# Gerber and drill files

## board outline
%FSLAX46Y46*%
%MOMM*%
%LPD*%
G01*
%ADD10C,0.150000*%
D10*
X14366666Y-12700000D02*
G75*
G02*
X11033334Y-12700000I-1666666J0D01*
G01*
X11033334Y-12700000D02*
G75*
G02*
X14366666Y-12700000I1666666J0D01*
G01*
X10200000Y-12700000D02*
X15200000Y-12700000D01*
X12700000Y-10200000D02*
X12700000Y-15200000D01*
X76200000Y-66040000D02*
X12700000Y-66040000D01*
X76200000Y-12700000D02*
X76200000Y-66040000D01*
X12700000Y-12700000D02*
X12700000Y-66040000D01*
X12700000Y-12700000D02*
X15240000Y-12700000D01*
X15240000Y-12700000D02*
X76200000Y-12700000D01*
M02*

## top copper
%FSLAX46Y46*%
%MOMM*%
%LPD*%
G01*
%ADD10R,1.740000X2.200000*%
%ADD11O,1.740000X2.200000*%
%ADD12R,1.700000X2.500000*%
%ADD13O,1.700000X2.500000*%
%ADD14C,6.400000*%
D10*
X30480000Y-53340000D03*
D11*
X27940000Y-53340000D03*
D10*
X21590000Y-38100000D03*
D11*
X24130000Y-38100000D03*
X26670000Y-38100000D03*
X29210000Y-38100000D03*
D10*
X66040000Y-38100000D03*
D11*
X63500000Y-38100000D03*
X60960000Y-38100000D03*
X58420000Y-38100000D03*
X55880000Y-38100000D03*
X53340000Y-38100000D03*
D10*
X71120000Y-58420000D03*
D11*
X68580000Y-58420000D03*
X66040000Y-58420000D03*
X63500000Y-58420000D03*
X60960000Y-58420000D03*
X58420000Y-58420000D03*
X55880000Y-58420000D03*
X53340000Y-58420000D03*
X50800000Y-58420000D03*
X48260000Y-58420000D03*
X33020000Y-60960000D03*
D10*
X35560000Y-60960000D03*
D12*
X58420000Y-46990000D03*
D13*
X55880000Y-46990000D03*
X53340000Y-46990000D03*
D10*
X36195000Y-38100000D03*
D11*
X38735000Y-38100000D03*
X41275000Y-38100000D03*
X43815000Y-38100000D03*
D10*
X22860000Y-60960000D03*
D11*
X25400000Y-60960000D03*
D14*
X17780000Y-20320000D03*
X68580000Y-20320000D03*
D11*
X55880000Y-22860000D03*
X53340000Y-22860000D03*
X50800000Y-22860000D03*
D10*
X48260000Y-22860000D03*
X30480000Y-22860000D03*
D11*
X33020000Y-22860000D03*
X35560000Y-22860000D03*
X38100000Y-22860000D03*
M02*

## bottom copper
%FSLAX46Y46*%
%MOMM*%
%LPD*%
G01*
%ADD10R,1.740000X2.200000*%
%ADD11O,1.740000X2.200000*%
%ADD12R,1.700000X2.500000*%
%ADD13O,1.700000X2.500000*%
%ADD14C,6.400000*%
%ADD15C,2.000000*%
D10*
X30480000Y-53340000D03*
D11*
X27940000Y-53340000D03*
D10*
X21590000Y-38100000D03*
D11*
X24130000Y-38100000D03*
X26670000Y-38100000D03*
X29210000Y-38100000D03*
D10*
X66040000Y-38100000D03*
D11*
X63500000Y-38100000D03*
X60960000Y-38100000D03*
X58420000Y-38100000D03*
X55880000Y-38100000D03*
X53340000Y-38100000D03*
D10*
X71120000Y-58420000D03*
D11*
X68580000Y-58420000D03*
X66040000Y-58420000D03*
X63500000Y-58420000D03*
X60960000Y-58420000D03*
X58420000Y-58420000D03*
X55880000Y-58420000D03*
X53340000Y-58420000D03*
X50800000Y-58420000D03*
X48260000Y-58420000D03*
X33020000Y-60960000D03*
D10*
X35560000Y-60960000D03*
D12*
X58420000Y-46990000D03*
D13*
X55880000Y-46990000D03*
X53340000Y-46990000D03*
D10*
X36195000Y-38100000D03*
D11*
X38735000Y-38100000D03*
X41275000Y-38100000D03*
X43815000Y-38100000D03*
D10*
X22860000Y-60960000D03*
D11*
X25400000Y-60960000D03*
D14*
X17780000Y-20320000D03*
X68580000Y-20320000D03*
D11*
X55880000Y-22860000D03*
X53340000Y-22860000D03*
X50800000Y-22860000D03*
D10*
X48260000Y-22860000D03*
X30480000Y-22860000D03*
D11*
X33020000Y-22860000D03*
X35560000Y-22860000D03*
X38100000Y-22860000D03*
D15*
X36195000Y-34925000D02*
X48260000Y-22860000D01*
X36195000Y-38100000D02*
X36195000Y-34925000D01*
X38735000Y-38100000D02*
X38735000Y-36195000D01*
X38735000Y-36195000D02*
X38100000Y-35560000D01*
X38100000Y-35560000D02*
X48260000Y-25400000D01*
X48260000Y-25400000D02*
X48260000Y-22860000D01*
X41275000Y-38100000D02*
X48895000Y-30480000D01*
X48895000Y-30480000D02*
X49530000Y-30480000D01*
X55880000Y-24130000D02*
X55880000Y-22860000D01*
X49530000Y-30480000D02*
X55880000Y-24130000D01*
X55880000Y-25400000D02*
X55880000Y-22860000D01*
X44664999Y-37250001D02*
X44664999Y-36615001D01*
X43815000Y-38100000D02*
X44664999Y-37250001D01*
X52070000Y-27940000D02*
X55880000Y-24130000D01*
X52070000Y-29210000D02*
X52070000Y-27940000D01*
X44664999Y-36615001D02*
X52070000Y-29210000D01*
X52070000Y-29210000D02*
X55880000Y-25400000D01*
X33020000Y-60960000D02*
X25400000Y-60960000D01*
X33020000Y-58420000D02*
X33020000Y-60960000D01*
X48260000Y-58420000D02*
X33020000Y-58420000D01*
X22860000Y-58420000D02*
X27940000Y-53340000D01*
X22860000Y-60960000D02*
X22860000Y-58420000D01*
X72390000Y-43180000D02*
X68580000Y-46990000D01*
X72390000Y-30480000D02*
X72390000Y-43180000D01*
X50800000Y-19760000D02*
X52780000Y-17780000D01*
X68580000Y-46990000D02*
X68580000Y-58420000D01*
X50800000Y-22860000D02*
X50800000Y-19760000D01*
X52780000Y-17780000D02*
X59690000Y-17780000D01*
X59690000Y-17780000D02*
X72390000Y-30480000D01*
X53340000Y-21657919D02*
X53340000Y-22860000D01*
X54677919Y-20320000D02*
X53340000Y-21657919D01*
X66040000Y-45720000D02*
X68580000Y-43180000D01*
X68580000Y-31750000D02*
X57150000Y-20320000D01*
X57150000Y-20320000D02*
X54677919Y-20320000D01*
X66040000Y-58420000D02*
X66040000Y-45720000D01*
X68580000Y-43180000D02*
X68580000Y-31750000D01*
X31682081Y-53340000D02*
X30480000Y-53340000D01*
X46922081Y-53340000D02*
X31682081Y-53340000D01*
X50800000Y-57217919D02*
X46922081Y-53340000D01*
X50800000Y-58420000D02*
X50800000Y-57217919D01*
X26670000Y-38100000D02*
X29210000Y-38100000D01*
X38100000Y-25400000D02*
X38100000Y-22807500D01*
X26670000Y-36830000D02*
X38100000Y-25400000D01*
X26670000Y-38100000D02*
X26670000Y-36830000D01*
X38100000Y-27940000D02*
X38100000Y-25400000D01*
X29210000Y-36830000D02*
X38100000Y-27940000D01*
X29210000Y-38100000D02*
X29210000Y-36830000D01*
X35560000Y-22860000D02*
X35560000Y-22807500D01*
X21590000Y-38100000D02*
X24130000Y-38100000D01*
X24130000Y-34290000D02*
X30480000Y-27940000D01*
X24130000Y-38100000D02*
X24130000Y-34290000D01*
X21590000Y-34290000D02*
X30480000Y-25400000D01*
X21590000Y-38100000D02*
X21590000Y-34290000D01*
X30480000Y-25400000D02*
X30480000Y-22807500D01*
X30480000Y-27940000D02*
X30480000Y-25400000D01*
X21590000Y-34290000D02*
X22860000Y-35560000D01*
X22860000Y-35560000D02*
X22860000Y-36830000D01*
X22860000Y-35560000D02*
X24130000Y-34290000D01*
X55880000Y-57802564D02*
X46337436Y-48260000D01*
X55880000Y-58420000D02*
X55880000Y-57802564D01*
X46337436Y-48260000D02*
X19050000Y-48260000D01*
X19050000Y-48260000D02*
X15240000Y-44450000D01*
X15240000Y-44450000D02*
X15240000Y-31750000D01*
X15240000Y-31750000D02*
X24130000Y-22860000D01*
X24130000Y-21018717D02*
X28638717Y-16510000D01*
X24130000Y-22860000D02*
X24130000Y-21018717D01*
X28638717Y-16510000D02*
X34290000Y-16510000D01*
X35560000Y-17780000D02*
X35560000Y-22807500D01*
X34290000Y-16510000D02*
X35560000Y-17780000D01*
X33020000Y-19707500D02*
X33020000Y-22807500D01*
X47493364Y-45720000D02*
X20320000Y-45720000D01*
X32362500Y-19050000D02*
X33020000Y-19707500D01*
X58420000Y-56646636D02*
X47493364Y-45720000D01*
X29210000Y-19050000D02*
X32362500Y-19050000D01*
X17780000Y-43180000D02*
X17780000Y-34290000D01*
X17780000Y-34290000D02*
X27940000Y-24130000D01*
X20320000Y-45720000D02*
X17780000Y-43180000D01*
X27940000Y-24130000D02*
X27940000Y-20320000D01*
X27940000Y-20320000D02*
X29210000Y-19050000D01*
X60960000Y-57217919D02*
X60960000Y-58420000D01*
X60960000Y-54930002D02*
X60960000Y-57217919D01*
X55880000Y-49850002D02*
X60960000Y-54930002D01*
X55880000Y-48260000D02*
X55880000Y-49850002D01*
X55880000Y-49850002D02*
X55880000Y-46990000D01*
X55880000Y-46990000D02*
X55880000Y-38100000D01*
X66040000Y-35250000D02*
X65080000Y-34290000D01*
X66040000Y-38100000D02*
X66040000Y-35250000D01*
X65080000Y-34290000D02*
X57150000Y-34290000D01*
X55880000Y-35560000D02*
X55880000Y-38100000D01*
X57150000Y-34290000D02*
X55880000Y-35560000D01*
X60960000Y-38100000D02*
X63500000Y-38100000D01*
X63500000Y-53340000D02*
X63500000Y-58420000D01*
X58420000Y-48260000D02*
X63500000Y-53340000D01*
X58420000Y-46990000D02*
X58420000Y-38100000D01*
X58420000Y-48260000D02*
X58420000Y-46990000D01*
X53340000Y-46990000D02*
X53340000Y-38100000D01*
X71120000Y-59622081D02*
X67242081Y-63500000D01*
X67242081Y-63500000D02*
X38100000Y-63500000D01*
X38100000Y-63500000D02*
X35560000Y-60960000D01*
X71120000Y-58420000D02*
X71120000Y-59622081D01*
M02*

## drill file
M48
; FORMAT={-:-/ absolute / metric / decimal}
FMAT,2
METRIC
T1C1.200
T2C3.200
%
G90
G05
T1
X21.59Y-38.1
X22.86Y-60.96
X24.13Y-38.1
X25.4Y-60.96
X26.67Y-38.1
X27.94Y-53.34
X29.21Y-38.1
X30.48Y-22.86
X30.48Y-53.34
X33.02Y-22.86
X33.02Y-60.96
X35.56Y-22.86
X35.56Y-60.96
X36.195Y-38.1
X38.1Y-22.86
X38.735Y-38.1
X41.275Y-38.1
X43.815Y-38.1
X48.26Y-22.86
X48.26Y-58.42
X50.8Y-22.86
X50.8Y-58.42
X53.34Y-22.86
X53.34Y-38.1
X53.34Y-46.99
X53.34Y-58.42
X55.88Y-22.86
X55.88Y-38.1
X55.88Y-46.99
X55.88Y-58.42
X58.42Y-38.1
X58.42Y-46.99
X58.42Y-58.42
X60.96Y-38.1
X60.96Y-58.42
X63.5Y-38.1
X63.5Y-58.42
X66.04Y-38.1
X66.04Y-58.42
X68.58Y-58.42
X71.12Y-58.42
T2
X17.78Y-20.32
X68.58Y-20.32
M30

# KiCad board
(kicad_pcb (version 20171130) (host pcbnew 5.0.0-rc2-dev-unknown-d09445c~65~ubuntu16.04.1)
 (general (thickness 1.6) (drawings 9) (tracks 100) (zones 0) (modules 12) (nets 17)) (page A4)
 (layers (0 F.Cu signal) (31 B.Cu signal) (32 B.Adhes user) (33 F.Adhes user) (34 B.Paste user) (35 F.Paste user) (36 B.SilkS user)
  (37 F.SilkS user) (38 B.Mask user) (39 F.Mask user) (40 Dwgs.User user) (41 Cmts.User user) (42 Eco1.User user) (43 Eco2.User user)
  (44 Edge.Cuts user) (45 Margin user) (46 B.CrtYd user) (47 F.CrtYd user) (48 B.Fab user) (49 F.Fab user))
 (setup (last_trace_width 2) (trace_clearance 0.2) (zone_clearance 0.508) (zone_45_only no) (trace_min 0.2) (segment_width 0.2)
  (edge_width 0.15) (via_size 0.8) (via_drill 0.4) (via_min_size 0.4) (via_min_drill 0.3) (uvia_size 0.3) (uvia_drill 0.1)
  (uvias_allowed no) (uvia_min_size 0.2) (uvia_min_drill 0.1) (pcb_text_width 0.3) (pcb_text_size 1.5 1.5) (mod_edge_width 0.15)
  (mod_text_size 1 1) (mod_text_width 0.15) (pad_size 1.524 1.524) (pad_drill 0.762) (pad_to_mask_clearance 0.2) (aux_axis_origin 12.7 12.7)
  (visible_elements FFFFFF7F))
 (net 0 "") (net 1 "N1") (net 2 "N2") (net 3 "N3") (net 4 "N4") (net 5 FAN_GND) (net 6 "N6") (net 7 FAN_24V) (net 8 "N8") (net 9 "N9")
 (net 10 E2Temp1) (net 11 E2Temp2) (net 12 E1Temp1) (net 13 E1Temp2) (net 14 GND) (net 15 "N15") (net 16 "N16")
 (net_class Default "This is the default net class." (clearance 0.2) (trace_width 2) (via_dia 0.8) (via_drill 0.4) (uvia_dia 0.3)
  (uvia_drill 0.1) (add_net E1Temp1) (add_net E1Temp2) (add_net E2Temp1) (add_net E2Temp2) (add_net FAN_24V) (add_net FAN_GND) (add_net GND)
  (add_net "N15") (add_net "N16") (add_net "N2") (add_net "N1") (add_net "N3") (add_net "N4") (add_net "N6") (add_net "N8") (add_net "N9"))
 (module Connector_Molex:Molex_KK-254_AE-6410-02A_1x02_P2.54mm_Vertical (layer F.Cu) (at 30.48 53.34 180)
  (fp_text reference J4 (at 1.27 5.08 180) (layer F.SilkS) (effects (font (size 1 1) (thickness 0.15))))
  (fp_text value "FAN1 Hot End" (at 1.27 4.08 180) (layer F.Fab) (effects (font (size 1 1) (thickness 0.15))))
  (pad 1 thru_hole rect (at 0 0 180) (size 1.74 2.2) (drill 1.2) (layers *.Cu *.Mask) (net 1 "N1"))
  (pad 2 thru_hole oval (at 2.54 0 180) (size 1.74 2.2) (drill 1.2) (layers *.Cu *.Mask) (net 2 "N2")))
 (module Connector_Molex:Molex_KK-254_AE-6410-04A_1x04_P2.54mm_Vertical (layer F.Cu) (at 21.59 38.1)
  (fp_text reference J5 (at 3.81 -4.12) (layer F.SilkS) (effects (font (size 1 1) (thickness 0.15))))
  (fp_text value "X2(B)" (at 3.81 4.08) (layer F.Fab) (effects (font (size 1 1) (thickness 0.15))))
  (pad 1 thru_hole rect (at 0 0) (size 1.74 2.2) (drill 1.2) (layers *.Cu *.Mask) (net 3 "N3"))
  (pad 2 thru_hole oval (at 2.54 0) (size 1.74 2.2) (drill 1.2) (layers *.Cu *.Mask) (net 3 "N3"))
  (pad 3 thru_hole oval (at 5.08 0) (size 1.74 2.2) (drill 1.2) (layers *.Cu *.Mask) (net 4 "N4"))
  (pad 4 thru_hole oval (at 7.62 0) (size 1.74 2.2) (drill 1.2) (layers *.Cu *.Mask) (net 4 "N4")))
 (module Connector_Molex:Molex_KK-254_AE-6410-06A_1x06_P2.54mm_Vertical (layer F.Cu) (at 66.04 38.1 180)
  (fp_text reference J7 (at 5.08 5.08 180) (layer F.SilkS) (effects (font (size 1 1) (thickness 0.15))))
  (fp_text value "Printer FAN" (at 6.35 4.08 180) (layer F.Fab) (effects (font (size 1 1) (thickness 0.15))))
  (pad 1 thru_hole rect (at 0 0 180) (size 1.74 2.2) (drill 1.2) (layers *.Cu *.Mask) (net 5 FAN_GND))
  (pad 2 thru_hole oval (at 2.54 0 180) (size 1.74 2.2) (drill 1.2) (layers *.Cu *.Mask) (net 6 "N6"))
  (pad 3 thru_hole oval (at 5.08 0 180) (size 1.74 2.2) (drill 1.2) (layers *.Cu *.Mask) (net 6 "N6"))
  (pad 4 thru_hole oval (at 7.62 0 180) (size 1.74 2.2) (drill 1.2) (layers *.Cu *.Mask) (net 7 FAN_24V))
  (pad 5 thru_hole oval (at 10.16 0 180) (size 1.74 2.2) (drill 1.2) (layers *.Cu *.Mask) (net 5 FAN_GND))
  (pad 6 thru_hole oval (at 12.7 0 180) (size 1.74 2.2) (drill 1.2) (layers *.Cu *.Mask) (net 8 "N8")))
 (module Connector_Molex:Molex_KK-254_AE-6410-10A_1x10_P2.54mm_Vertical (layer F.Cu) (at 71.12 58.42 180)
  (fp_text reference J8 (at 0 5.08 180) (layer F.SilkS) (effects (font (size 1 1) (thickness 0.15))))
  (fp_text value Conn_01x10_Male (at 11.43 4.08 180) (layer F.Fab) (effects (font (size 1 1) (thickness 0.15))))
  (pad 1 thru_hole rect (at 0 0 180) (size 1.74 2.2) (drill 1.2) (layers *.Cu *.Mask) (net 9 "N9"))
  (pad 2 thru_hole oval (at 2.54 0 180) (size 1.74 2.2) (drill 1.2) (layers *.Cu *.Mask) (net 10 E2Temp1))
  (pad 3 thru_hole oval (at 5.08 0 180) (size 1.74 2.2) (drill 1.2) (layers *.Cu *.Mask) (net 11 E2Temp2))
  (pad 4 thru_hole oval (at 7.62 0 180) (size 1.74 2.2) (drill 1.2) (layers *.Cu *.Mask) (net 7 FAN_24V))
  (pad 5 thru_hole oval (at 10.16 0 180) (size 1.74 2.2) (drill 1.2) (layers *.Cu *.Mask) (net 5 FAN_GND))
  (pad 6 thru_hole oval (at 12.7 0 180) (size 1.74 2.2) (drill 1.2) (layers *.Cu *.Mask) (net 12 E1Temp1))
  (pad 7 thru_hole oval (at 15.24 0 180) (size 1.74 2.2) (drill 1.2) (layers *.Cu *.Mask) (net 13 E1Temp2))
  (pad 8 thru_hole oval (at 17.78 0 180) (size 1.74 2.2) (drill 1.2) (layers *.Cu *.Mask))
  (pad 9 thru_hole oval (at 20.32 0 180) (size 1.74 2.2) (drill 1.2) (layers *.Cu *.Mask) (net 1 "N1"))
  (pad 10 thru_hole oval (at 22.86 0 180) (size 1.74 2.2) (drill 1.2) (layers *.Cu *.Mask) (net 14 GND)))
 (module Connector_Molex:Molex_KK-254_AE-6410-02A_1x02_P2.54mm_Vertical (layer F.Cu) (at 35.56 60.96 180)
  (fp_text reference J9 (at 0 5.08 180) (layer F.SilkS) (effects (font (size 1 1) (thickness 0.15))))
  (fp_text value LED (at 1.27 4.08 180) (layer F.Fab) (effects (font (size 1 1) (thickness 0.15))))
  (pad 2 thru_hole oval (at 2.54 0 180) (size 1.74 2.2) (drill 1.2) (layers *.Cu *.Mask) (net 14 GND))
  (pad 1 thru_hole rect (at 0 0 180) (size 1.74 2.2) (drill 1.2) (layers *.Cu *.Mask) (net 9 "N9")))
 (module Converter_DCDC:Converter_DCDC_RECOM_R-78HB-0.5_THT (layer F.Cu) (at 58.42 46.99 180)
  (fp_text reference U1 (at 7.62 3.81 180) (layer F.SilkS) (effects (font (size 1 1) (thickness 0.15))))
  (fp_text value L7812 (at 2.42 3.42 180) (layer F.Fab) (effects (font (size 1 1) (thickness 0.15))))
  (pad 1 thru_hole rect (at 0 0 180) (size 1.7 2.5) (drill 1.2) (layers *.Cu *.Mask) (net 7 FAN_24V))
  (pad 2 thru_hole oval (at 2.54 0 180) (size 1.7 2.5) (drill 1.2) (layers *.Cu *.Mask) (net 5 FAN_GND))
  (pad 3 thru_hole oval (at 5.08 0 180) (size 1.7 2.5) (drill 1.2) (layers *.Cu *.Mask) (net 8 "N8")))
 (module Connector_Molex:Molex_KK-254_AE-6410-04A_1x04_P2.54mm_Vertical (layer F.Cu) (at 36.195 38.1)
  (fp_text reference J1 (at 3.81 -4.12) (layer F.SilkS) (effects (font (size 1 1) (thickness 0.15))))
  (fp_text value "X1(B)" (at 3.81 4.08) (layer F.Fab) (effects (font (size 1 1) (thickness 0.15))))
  (pad 1 thru_hole rect (at 0 0) (size 1.74 2.2) (drill 1.2) (layers *.Cu *.Mask) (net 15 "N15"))
  (pad 2 thru_hole oval (at 2.54 0) (size 1.74 2.2) (drill 1.2) (layers *.Cu *.Mask) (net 15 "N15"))
  (pad 3 thru_hole oval (at 5.08 0) (size 1.74 2.2) (drill 1.2) (layers *.Cu *.Mask) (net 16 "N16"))
  (pad 4 thru_hole oval (at 7.62 0) (size 1.74 2.2) (drill 1.2) (layers *.Cu *.Mask) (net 16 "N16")))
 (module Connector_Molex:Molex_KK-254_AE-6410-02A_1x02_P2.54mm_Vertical (layer F.Cu) (at 22.86 60.96)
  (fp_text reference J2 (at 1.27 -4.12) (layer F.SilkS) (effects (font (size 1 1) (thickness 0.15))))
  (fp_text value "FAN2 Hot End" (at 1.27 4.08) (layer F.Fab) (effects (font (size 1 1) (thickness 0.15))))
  (pad 1 thru_hole rect (at 0 0) (size 1.74 2.2) (drill 1.2) (layers *.Cu *.Mask) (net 2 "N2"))
  (pad 2 thru_hole oval (at 2.54 0) (size 1.74 2.2) (drill 1.2) (layers *.Cu *.Mask) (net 14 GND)))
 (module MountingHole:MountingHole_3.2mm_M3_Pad (layer F.Cu) (at 17.78 20.32)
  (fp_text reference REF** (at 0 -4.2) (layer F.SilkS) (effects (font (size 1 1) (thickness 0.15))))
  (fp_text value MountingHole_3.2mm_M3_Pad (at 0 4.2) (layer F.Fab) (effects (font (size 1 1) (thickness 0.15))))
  (pad 1 thru_hole circle (at 0 0) (size 6.4 6.4) (drill 3.2) (layers *.Cu *.Mask)))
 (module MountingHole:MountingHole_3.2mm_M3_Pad (layer F.Cu) (at 68.58 20.32)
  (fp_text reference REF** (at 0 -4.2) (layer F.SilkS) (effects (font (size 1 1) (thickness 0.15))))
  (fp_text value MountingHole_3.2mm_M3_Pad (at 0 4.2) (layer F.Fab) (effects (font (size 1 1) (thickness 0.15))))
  (pad 1 thru_hole circle (at 0 0) (size 6.4 6.4) (drill 3.2) (layers *.Cu *.Mask)))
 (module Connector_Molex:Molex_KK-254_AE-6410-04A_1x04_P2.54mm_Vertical (layer F.Cu) (at 48.26 22.86)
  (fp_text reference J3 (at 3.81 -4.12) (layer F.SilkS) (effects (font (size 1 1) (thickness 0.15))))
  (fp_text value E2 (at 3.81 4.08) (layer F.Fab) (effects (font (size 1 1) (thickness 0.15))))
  (pad 4 thru_hole oval (at 7.62 0) (size 1.74 2.2) (drill 1.2) (layers *.Cu *.Mask) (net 16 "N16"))
  (pad 3 thru_hole oval (at 5.08 0) (size 1.74 2.2) (drill 1.2) (layers *.Cu *.Mask) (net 11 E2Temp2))
  (pad 2 thru_hole oval (at 2.54 0) (size 1.74 2.2) (drill 1.2) (layers *.Cu *.Mask) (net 10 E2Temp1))
  (pad 1 thru_hole rect (at 0 0) (size 1.74 2.2) (drill 1.2) (layers *.Cu *.Mask) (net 15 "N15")))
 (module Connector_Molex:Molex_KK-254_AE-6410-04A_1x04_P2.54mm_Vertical (layer F.Cu) (at 30.48 22.86)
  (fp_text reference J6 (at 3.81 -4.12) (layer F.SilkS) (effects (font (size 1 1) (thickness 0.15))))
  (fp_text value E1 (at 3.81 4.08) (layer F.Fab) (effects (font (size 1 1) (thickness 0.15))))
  (pad 1 thru_hole rect (at 0 0) (size 1.74 2.2) (drill 1.2) (layers *.Cu *.Mask) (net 3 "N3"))
  (pad 2 thru_hole oval (at 2.54 0) (size 1.74 2.2) (drill 1.2) (layers *.Cu *.Mask) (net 12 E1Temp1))
  (pad 3 thru_hole oval (at 5.08 0) (size 1.74 2.2) (drill 1.2) (layers *.Cu *.Mask) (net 13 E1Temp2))
  (pad 4 thru_hole oval (at 7.62 0) (size 1.74 2.2) (drill 1.2) (layers *.Cu *.Mask) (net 4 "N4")))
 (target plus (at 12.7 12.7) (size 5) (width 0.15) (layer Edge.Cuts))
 (gr_line (start 76.2 66.04) (end 12.7 66.04) (layer Edge.Cuts) (width 0.15))
 (gr_line (start 76.2 12.7) (end 76.2 66.04) (layer Edge.Cuts) (width 0.15))
 (gr_line (start 12.7 12.7) (end 12.7 66.04) (layer Edge.Cuts) (width 0.15))
 (gr_line (start 12.7 12.7) (end 15.24 12.7) (layer Edge.Cuts) (width 0.15))
 (gr_line (start 15.24 12.7) (end 76.2 12.7) (layer Edge.Cuts) (width 0.15))
 (segment (start 36.195 34.925) (end 48.26 22.86) (width 2) (layer B.Cu) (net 15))
 (segment (start 36.195 38.1) (end 36.195 34.925) (width 2) (layer B.Cu) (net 15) (status 10))
 (segment (start 38.735 38.1) (end 38.735 36.195) (width 2) (layer B.Cu) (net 15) (status 10))
 (segment (start 38.735 36.195) (end 38.1 35.56) (width 2) (layer B.Cu) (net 15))
 (segment (start 38.1 35.56) (end 48.26 25.4) (width 2) (layer B.Cu) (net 15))
 (segment (start 48.26 25.4) (end 48.26 22.86) (width 2) (layer B.Cu) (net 15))
 (segment (start 41.275 38.1) (end 48.895 30.48) (width 2) (layer B.Cu) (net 16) (status 10))
 (segment (start 48.895 30.48) (end 49.53 30.48) (width 2) (layer B.Cu) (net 16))
 (segment (start 55.88 24.13) (end 55.88 22.86) (width 2) (layer B.Cu) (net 16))
 (segment (start 49.53 30.48) (end 55.88 24.13) (width 2) (layer B.Cu) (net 16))
 (segment (start 55.88 25.4) (end 55.88 22.86) (width 2) (layer B.Cu) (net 16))
 (segment (start 44.664999 37.250001) (end 44.664999 36.615001) (width 2) (layer B.Cu) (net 16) (status 10))
 (segment (start 43.815 38.1) (end 44.664999 37.250001) (width 2) (layer B.Cu) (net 16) (status 30))
 (segment (start 52.07 27.94) (end 55.88 24.13) (width 2) (layer B.Cu) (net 16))
 (segment (start 52.07 29.21) (end 52.07 27.94) (width 2) (layer B.Cu) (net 16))
 (segment (start 44.664999 36.615001) (end 52.07 29.21) (width 2) (layer B.Cu) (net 16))
 (segment (start 52.07 29.21) (end 55.88 25.4) (width 2) (layer B.Cu) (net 16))
 (segment (start 33.02 60.96) (end 25.4 60.96) (width 2) (layer B.Cu) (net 14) (status 30))
 (segment (start 33.02 58.42) (end 33.02 60.96) (width 2) (layer B.Cu) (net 14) (status 20))
 (segment (start 48.26 58.42) (end 33.02 58.42) (width 2) (layer B.Cu) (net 14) (status 10))
 (segment (start 22.86 58.42) (end 27.94 53.34) (width 2) (layer B.Cu) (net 2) (status 20))
 (segment (start 22.86 60.96) (end 22.86 58.42) (width 2) (layer B.Cu) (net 2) (status 10))
 (segment (start 72.39 43.18) (end 68.58 46.99) (width 2) (layer B.Cu) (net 10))
 (segment (start 72.39 30.48) (end 72.39 43.18) (width 2) (layer B.Cu) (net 10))
 (segment (start 50.8 19.76) (end 52.78 17.78) (width 2) (layer B.Cu) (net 10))
 (segment (start 68.58 46.99) (end 68.58 58.42) (width 2) (layer B.Cu) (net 10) (status 20))
 (segment (start 50.8 22.86) (end 50.8 19.76) (width 2) (layer B.Cu) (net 10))
 (segment (start 52.78 17.78) (end 59.69 17.78) (width 2) (layer B.Cu) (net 10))
 (segment (start 59.69 17.78) (end 72.39 30.48) (width 2) (layer B.Cu) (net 10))
 (segment (start 53.34 21.657919) (end 53.34 22.86) (width 2) (layer B.Cu) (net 11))
 (segment (start 54.677919 20.32) (end 53.34 21.657919) (width 2) (layer B.Cu) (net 11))
 (segment (start 66.04 45.72) (end 68.58 43.18) (width 2) (layer B.Cu) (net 11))
 (segment (start 68.58 31.75) (end 57.15 20.32) (width 2) (layer B.Cu) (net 11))
 (segment (start 57.15 20.32) (end 54.677919 20.32) (width 2) (layer B.Cu) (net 11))
 (segment (start 66.04 58.42) (end 66.04 45.72) (width 2) (layer B.Cu) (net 11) (status 10))
 (segment (start 68.58 43.18) (end 68.58 31.75) (width 2) (layer B.Cu) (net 11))
 (segment (start 31.682081 53.34) (end 30.48 53.34) (width 2) (layer B.Cu) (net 1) (status 20))
 (segment (start 46.922081 53.34) (end 31.682081 53.34) (width 2) (layer B.Cu) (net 1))
 (segment (start 50.8 57.217919) (end 46.922081 53.34) (width 2) (layer B.Cu) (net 1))
 (segment (start 50.8 58.42) (end 50.8 57.217919) (width 2) (layer B.Cu) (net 1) (status 10))
 (segment (start 26.67 38.1) (end 29.21 38.1) (width 2) (layer B.Cu) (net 4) (status 30))
 (segment (start 38.1 25.4) (end 38.1 22.8075) (width 2) (layer B.Cu) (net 4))
 (segment (start 26.67 36.83) (end 38.1 25.4) (width 2) (layer B.Cu) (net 4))
 (segment (start 26.67 38.1) (end 26.67 36.83) (width 2) (layer B.Cu) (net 4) (status 10))
 (segment (start 38.1 27.94) (end 38.1 25.4) (width 2) (layer B.Cu) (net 4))
 (segment (start 29.21 36.83) (end 38.1 27.94) (width 2) (layer B.Cu) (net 4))
 (segment (start 29.21 38.1) (end 29.21 36.83) (width 2) (layer B.Cu) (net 4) (status 10))
 (segment (start 35.56 22.86) (end 35.56 22.8075) (width 2) (layer B.Cu) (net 13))
 (segment (start 21.59 38.1) (end 24.13 38.1) (width 2) (layer B.Cu) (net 3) (status 30))
 (segment (start 24.13 34.29) (end 30.48 27.94) (width 2) (layer B.Cu) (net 3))
 (segment (start 24.13 38.1) (end 24.13 34.29) (width 2) (layer B.Cu) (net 3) (status 10))
 (segment (start 21.59 34.29) (end 30.48 25.4) (width 2) (layer B.Cu) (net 3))
 (segment (start 21.59 38.1) (end 21.59 34.29) (width 2) (layer B.Cu) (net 3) (status 10))
 (segment (start 30.48 25.4) (end 30.48 22.8075) (width 2) (layer B.Cu) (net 3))
 (segment (start 30.48 27.94) (end 30.48 25.4) (width 2) (layer B.Cu) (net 3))
 (segment (start 21.59 34.29) (end 22.86 35.56) (width 2) (layer B.Cu) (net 3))
 (segment (start 22.86 35.56) (end 22.86 36.83) (width 2) (layer B.Cu) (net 3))
 (segment (start 22.86 35.56) (end 24.13 34.29) (width 2) (layer B.Cu) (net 3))
 (segment (start 55.88 57.802564) (end 46.337436 48.26) (width 2) (layer B.Cu) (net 13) (status 10))
 (segment (start 55.88 58.42) (end 55.88 57.802564) (width 2) (layer B.Cu) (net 13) (status 30))
 (segment (start 46.337436 48.26) (end 19.05 48.26) (width 2) (layer B.Cu) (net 13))
 (segment (start 19.05 48.26) (end 15.24 44.45) (width 2) (layer B.Cu) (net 13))
 (segment (start 15.24 44.45) (end 15.24 31.75) (width 2) (layer B.Cu) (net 13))
 (segment (start 15.24 31.75) (end 24.13 22.86) (width 2) (layer B.Cu) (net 13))
 (segment (start 24.13 21.018717) (end 28.638717 16.51) (width 2) (layer B.Cu) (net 13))
 (segment (start 24.13 22.86) (end 24.13 21.018717) (width 2) (layer B.Cu) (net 13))
 (segment (start 28.638717 16.51) (end 34.29 16.51) (width 2) (layer B.Cu) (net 13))
 (segment (start 35.56 17.78) (end 35.56 22.8075) (width 2) (layer B.Cu) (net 13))
 (segment (start 34.29 16.51) (end 35.56 17.78) (width 2) (layer B.Cu) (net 13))
 (segment (start 33.02 19.7075) (end 33.02 22.8075) (width 2) (layer B.Cu) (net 12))
 (segment (start 47.493364 45.72) (end 20.32 45.72) (width 2) (layer B.Cu) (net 12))
 (segment (start 32.3625 19.05) (end 33.02 19.7075) (width 2) (layer B.Cu) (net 12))
 (segment (start 58.42 56.646636) (end 47.493364 45.72) (width 2) (layer B.Cu) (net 12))
 (segment (start 29.21 19.05) (end 32.3625 19.05) (width 2) (layer B.Cu) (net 12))
 (segment (start 17.78 43.18) (end 17.78 34.29) (width 2) (layer B.Cu) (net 12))
 (segment (start 17.78 34.29) (end 27.94 24.13) (width 2) (layer B.Cu) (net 12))
 (segment (start 20.32 45.72) (end 17.78 43.18) (width 2) (layer B.Cu) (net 12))
 (segment (start 27.94 24.13) (end 27.94 20.32) (width 2) (layer B.Cu) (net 12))
 (segment (start 27.94 20.32) (end 29.21 19.05) (width 2) (layer B.Cu) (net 12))
 (segment (start 60.96 57.217919) (end 60.96 58.42) (width 2) (layer B.Cu) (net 5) (status 20))
 (segment (start 60.96 54.930002) (end 60.96 57.217919) (width 2) (layer B.Cu) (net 5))
 (segment (start 55.88 49.850002) (end 60.96 54.930002) (width 2) (layer B.Cu) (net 5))
 (segment (start 55.88 48.26) (end 55.88 49.850002) (width 2) (layer B.Cu) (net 5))
 (segment (start 55.88 49.850002) (end 55.88 46.99) (width 2) (layer B.Cu) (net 5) (status 20))
 (segment (start 55.88 46.99) (end 55.88 38.1) (width 2) (layer B.Cu) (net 5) (status 30))
 (segment (start 66.04 35.25) (end 65.08 34.29) (width 2) (layer B.Cu) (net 5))
 (segment (start 66.04 38.1) (end 66.04 35.25) (width 2) (layer B.Cu) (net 5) (status 10))
 (segment (start 65.08 34.29) (end 57.15 34.29) (width 2) (layer B.Cu) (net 5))
 (segment (start 55.88 35.56) (end 55.88 38.1) (width 2) (layer B.Cu) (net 5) (status 20))
 (segment (start 57.15 34.29) (end 55.88 35.56) (width 2) (layer B.Cu) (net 5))
 (segment (start 60.96 38.1) (end 63.5 38.1) (width 2) (layer B.Cu) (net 6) (status 30))
 (segment (start 63.5 53.34) (end 63.5 58.42) (width 2) (layer B.Cu) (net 7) (status 20))
 (segment (start 58.42 48.26) (end 63.5 53.34) (width 2) (layer B.Cu) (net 7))
 (segment (start 58.42 46.99) (end 58.42 38.1) (width 2) (layer B.Cu) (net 7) (status 30))
 (segment (start 58.42 48.26) (end 58.42 46.99) (width 2) (layer B.Cu) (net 7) (status 20))
 (segment (start 53.34 46.99) (end 53.34 38.1) (width 2) (layer B.Cu) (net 8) (status 30))
 (segment (start 71.12 59.622081) (end 67.242081 63.5) (width 2) (layer B.Cu) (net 9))
 (segment (start 67.242081 63.5) (end 38.1 63.5) (width 2) (layer B.Cu) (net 9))
 (segment (start 38.1 63.5) (end 35.56 60.96) (width 2) (layer B.Cu) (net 9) (status 20))
 (segment (start 71.12 58.42) (end 71.12 59.622081) (width 2) (layer B.Cu) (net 9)))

